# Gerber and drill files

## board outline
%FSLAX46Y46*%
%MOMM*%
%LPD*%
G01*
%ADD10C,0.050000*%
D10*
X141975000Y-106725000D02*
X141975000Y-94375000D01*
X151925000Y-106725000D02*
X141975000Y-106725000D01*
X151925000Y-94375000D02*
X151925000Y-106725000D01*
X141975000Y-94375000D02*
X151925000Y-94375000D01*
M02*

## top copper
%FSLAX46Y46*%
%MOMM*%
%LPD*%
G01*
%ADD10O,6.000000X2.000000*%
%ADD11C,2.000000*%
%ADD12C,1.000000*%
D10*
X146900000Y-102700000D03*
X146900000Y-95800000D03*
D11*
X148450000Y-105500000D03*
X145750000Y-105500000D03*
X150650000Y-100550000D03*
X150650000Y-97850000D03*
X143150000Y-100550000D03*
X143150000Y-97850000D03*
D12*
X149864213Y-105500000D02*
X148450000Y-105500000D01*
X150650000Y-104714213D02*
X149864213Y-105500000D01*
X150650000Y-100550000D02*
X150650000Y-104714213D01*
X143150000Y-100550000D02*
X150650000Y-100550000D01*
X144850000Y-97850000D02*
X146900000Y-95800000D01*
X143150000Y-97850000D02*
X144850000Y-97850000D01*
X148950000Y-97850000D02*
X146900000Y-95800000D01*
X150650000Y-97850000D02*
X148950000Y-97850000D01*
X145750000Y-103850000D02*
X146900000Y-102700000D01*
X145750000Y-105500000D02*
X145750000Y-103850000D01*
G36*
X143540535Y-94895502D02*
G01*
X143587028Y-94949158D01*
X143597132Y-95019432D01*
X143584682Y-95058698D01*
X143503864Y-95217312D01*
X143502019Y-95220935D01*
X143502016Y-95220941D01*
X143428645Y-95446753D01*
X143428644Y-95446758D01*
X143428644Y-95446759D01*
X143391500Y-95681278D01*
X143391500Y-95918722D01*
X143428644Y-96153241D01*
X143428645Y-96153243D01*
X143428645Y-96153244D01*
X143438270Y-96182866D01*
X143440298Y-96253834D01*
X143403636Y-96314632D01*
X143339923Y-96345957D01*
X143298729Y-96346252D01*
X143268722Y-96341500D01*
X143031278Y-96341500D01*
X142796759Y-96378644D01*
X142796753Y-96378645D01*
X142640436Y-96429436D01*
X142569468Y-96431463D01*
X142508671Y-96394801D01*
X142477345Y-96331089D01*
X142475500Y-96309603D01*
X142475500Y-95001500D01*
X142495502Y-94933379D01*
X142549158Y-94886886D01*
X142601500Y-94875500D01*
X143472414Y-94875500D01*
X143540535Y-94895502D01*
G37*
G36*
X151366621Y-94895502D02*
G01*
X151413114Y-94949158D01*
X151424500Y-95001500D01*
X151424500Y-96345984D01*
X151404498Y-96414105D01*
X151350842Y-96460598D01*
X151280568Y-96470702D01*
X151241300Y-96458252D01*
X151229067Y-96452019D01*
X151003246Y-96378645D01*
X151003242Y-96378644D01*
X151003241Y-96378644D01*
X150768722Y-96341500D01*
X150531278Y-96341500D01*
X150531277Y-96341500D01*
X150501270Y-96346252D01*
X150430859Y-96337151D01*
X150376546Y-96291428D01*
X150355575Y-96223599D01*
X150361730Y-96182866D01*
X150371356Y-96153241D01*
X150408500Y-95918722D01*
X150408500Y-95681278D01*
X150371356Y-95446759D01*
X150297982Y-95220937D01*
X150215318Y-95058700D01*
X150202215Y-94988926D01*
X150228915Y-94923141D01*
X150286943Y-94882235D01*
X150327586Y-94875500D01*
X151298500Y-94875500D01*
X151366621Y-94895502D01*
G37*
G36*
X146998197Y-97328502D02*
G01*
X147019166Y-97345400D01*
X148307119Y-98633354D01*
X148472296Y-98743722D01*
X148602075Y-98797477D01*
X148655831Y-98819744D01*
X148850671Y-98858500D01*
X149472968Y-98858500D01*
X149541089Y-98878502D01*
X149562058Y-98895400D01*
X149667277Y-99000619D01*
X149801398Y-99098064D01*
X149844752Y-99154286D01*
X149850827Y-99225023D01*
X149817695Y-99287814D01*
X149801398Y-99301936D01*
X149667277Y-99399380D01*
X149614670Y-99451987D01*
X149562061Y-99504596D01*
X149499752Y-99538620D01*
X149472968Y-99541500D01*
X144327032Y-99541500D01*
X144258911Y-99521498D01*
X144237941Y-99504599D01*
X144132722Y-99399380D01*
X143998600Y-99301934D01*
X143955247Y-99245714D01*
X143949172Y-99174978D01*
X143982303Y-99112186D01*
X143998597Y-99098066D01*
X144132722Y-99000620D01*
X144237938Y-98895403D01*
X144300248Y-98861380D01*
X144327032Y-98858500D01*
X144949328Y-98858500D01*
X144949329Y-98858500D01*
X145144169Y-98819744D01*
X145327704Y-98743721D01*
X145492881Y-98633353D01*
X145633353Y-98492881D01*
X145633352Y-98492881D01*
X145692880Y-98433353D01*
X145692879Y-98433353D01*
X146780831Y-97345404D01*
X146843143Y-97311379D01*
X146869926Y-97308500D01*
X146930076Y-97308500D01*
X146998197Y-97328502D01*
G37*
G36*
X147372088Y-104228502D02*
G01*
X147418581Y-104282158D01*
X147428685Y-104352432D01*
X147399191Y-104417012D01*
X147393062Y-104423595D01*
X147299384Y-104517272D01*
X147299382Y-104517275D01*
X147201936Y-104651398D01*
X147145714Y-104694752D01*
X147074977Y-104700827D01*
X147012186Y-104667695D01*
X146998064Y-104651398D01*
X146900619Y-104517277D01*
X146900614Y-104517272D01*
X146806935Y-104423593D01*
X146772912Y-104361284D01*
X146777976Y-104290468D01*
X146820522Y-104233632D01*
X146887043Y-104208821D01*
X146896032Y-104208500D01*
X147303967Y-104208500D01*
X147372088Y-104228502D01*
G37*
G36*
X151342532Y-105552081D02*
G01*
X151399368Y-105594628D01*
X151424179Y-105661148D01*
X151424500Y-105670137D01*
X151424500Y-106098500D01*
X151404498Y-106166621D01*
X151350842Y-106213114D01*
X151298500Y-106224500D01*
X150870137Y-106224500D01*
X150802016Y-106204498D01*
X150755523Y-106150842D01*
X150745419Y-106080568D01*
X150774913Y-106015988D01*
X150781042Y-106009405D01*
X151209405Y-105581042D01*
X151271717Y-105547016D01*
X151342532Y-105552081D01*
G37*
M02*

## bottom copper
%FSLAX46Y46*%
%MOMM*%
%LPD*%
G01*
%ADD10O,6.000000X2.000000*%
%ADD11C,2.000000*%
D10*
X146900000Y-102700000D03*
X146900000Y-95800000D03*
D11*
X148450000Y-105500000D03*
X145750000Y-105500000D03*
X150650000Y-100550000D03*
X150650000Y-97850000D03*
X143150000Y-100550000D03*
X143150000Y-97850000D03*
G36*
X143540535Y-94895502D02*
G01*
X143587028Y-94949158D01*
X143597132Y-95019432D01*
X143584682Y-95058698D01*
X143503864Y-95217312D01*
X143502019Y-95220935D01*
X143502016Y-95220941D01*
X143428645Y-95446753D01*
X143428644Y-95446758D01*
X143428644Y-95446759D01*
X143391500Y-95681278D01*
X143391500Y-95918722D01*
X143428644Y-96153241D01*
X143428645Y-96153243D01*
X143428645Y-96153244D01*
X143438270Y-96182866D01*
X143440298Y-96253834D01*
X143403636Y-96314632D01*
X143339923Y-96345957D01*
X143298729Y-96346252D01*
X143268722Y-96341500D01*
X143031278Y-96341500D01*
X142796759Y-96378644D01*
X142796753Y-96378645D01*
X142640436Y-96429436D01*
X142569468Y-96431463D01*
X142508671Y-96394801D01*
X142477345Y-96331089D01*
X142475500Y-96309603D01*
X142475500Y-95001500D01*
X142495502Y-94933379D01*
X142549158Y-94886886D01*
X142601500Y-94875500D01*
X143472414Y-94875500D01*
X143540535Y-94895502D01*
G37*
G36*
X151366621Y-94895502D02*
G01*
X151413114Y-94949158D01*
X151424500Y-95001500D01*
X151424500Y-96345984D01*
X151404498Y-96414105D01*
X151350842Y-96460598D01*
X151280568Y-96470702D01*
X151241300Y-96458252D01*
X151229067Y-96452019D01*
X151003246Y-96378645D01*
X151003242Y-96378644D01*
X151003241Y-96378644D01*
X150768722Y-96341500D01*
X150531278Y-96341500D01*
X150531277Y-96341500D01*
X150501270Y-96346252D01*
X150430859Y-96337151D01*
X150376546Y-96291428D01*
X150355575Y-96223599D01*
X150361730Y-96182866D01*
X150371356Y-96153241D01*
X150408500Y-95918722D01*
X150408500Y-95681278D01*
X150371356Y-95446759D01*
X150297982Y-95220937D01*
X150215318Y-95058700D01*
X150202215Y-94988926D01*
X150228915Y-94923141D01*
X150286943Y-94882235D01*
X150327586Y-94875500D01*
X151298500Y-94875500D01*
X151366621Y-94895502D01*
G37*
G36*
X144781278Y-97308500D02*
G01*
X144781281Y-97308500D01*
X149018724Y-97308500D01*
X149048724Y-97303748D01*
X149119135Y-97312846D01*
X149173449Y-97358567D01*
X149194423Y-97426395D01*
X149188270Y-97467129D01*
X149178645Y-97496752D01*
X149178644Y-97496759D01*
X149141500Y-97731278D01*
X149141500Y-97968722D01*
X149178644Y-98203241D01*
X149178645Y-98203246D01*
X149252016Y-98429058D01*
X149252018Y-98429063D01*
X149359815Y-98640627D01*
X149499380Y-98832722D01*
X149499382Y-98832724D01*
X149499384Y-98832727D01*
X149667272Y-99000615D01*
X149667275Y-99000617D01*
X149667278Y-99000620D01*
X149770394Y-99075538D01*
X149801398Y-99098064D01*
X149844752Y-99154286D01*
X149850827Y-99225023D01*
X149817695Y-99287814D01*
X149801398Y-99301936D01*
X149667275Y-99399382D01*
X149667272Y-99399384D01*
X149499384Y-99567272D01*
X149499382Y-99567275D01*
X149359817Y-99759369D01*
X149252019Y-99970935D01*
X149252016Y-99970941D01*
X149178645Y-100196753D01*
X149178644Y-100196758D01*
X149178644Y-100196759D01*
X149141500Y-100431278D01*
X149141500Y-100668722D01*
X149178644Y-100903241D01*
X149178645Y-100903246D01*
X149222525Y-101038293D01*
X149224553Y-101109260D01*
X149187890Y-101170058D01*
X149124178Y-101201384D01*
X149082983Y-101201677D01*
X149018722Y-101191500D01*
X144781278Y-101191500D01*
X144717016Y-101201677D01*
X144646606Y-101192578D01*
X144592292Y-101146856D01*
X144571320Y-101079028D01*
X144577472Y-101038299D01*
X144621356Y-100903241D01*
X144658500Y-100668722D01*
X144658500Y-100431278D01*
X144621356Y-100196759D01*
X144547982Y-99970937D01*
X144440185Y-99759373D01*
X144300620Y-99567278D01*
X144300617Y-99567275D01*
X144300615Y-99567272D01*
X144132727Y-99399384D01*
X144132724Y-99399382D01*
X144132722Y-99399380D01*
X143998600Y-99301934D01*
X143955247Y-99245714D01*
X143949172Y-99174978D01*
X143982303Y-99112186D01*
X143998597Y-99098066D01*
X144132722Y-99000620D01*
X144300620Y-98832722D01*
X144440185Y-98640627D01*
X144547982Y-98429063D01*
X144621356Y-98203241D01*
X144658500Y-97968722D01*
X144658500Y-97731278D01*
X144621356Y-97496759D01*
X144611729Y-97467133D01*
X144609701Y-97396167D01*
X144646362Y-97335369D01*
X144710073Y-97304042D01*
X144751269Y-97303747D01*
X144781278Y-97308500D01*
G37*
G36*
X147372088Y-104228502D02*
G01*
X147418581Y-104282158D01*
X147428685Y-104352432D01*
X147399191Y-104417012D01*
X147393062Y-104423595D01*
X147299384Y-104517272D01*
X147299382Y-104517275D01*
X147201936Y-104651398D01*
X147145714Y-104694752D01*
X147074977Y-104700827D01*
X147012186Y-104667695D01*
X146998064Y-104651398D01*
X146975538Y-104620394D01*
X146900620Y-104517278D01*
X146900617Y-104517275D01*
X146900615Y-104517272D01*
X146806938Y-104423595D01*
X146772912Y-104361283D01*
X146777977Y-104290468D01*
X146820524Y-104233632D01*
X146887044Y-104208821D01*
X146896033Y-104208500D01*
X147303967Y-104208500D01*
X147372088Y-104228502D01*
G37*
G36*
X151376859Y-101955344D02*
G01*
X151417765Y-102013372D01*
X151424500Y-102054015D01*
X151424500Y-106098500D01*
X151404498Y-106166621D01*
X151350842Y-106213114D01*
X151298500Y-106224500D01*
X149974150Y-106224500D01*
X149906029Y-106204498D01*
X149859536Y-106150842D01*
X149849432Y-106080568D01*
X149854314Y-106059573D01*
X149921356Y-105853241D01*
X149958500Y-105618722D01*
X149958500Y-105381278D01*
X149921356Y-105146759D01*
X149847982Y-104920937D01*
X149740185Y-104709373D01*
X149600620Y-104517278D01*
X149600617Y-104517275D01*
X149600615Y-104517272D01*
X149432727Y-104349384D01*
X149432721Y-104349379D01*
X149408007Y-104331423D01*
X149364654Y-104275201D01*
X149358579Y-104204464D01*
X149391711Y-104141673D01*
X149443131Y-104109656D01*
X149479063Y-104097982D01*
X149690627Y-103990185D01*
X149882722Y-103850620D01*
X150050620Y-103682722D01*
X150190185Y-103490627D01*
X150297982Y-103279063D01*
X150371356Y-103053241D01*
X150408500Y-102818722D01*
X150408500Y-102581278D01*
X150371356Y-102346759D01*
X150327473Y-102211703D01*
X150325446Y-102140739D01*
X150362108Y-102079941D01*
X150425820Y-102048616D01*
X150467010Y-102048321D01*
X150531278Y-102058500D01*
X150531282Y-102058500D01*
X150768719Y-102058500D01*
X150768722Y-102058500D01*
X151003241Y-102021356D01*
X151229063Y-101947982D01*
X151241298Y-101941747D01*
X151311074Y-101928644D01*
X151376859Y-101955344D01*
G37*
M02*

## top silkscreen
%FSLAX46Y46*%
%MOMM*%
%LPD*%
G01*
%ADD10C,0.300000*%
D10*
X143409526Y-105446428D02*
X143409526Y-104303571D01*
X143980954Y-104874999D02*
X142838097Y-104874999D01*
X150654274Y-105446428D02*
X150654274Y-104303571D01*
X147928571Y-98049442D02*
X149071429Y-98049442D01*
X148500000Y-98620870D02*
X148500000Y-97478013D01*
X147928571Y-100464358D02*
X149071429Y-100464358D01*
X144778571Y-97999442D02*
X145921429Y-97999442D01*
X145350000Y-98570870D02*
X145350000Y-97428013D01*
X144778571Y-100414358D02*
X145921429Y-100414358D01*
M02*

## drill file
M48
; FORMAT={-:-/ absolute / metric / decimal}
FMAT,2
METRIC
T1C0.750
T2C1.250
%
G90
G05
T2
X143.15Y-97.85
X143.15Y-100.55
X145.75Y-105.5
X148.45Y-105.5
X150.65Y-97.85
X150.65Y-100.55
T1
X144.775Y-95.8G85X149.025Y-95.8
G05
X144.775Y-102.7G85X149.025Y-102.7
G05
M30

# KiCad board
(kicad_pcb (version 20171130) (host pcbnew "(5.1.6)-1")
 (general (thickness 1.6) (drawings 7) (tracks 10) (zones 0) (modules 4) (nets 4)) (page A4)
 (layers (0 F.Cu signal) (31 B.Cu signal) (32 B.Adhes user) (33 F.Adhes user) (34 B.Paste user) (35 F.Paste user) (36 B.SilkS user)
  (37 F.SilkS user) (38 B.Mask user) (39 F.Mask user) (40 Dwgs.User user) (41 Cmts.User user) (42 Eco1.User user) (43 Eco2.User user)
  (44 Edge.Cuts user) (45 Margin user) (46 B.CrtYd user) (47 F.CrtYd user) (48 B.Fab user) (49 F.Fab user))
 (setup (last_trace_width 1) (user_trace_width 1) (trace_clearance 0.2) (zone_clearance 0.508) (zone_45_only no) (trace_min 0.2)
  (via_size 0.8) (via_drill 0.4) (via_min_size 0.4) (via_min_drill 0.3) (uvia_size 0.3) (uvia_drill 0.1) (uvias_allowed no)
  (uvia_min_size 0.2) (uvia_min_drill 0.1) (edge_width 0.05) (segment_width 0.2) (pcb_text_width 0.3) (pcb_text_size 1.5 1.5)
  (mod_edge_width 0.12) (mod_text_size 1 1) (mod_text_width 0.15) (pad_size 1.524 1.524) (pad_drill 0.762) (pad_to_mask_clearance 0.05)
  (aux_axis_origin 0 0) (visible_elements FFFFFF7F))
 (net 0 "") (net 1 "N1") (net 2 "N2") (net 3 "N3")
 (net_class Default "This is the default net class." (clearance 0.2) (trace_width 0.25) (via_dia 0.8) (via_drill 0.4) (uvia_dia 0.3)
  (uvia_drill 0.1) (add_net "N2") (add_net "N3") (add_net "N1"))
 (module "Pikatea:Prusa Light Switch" (layer F.Cu) (at 146.9 95.8)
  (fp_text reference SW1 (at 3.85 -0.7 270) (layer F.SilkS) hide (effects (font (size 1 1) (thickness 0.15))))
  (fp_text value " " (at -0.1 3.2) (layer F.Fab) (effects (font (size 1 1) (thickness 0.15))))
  (pad 2 thru_hole oval (at 0 6.9) (size 6 2) (drill oval 5 0.75) (layers *.Cu *.Mask) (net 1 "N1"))
  (pad 1 thru_hole oval (at 0 0) (size 6 2) (drill oval 5 0.75) (layers *.Cu *.Mask) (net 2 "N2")))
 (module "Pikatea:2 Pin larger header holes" (layer F.Cu) (at 145.75 105.5 90)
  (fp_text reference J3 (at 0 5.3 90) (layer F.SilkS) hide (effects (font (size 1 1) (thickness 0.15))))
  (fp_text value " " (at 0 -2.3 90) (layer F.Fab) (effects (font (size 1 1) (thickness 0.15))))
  (pad 2 thru_hole circle (at 0 2.7 90) (size 2 2) (drill 1.25) (layers *.Cu *.Mask) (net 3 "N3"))
  (pad 1 thru_hole circle (at 0 0 90) (size 2 2) (drill 1.25) (layers *.Cu *.Mask) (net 1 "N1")))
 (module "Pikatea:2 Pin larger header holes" (layer F.Cu) (at 150.65 97.85)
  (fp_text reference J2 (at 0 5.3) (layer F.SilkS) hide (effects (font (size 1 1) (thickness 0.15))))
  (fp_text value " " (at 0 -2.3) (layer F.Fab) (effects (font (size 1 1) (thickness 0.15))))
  (pad 2 thru_hole circle (at 0 2.7) (size 2 2) (drill 1.25) (layers *.Cu *.Mask) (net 3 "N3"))
  (pad 1 thru_hole circle (at 0 0) (size 2 2) (drill 1.25) (layers *.Cu *.Mask) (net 2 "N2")))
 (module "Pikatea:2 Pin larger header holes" (layer F.Cu) (at 143.15 97.85)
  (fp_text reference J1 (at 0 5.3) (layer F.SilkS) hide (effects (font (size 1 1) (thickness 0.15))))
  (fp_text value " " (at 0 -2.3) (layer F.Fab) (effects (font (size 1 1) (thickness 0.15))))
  (pad 2 thru_hole circle (at 0 2.7) (size 2 2) (drill 1.25) (layers *.Cu *.Mask) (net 3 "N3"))
  (pad 1 thru_hole circle (at 0 0) (size 2 2) (drill 1.25) (layers *.Cu *.Mask) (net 2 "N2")))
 (gr_line (start 141.975 106.725) (end 141.975 94.375) (layer Edge.Cuts) (width 0.05))
 (gr_line (start 151.925 106.725) (end 141.975 106.725) (layer Edge.Cuts) (width 0.05))
 (gr_line (start 151.925 94.375) (end 151.925 106.725) (layer Edge.Cuts) (width 0.05))
 (gr_line (start 141.975 94.375) (end 151.925 94.375) (layer Edge.Cuts) (width 0.05))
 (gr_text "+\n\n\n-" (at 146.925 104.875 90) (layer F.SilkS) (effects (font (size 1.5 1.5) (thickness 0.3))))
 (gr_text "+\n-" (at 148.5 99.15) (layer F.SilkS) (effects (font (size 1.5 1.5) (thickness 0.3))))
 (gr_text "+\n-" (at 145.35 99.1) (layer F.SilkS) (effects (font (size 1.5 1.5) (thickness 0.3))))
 (segment (start 149.864213 105.5) (end 148.45 105.5) (width 1) (layer F.Cu) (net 3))
 (segment (start 150.65 104.714213) (end 149.864213 105.5) (width 1) (layer F.Cu) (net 3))
 (segment (start 150.65 100.55) (end 150.65 104.714213) (width 1) (layer F.Cu) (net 3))
 (segment (start 143.15 100.55) (end 150.65 100.55) (width 1) (layer F.Cu) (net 3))
 (segment (start 144.85 97.85) (end 146.9 95.8) (width 1) (layer F.Cu) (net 2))
 (segment (start 143.15 97.85) (end 144.85 97.85) (width 1) (layer F.Cu) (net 2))
 (segment (start 148.95 97.85) (end 146.9 95.8) (width 1) (layer F.Cu) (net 2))
 (segment (start 150.65 97.85) (end 148.95 97.85) (width 1) (layer F.Cu) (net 2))
 (segment (start 145.75 103.85) (end 146.9 102.7) (width 1) (layer F.Cu) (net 1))
 (segment (start 145.75 105.5) (end 145.75 103.85) (width 1) (layer F.Cu) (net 1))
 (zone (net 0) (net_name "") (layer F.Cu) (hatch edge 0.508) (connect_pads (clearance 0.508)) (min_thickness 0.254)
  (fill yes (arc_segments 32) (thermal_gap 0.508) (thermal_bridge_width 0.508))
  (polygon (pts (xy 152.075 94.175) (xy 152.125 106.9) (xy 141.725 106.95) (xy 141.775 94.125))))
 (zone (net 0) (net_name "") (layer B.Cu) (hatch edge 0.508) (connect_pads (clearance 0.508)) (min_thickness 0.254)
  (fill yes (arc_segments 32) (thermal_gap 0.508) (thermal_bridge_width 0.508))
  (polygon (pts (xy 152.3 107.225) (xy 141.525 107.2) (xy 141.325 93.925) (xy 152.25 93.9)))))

